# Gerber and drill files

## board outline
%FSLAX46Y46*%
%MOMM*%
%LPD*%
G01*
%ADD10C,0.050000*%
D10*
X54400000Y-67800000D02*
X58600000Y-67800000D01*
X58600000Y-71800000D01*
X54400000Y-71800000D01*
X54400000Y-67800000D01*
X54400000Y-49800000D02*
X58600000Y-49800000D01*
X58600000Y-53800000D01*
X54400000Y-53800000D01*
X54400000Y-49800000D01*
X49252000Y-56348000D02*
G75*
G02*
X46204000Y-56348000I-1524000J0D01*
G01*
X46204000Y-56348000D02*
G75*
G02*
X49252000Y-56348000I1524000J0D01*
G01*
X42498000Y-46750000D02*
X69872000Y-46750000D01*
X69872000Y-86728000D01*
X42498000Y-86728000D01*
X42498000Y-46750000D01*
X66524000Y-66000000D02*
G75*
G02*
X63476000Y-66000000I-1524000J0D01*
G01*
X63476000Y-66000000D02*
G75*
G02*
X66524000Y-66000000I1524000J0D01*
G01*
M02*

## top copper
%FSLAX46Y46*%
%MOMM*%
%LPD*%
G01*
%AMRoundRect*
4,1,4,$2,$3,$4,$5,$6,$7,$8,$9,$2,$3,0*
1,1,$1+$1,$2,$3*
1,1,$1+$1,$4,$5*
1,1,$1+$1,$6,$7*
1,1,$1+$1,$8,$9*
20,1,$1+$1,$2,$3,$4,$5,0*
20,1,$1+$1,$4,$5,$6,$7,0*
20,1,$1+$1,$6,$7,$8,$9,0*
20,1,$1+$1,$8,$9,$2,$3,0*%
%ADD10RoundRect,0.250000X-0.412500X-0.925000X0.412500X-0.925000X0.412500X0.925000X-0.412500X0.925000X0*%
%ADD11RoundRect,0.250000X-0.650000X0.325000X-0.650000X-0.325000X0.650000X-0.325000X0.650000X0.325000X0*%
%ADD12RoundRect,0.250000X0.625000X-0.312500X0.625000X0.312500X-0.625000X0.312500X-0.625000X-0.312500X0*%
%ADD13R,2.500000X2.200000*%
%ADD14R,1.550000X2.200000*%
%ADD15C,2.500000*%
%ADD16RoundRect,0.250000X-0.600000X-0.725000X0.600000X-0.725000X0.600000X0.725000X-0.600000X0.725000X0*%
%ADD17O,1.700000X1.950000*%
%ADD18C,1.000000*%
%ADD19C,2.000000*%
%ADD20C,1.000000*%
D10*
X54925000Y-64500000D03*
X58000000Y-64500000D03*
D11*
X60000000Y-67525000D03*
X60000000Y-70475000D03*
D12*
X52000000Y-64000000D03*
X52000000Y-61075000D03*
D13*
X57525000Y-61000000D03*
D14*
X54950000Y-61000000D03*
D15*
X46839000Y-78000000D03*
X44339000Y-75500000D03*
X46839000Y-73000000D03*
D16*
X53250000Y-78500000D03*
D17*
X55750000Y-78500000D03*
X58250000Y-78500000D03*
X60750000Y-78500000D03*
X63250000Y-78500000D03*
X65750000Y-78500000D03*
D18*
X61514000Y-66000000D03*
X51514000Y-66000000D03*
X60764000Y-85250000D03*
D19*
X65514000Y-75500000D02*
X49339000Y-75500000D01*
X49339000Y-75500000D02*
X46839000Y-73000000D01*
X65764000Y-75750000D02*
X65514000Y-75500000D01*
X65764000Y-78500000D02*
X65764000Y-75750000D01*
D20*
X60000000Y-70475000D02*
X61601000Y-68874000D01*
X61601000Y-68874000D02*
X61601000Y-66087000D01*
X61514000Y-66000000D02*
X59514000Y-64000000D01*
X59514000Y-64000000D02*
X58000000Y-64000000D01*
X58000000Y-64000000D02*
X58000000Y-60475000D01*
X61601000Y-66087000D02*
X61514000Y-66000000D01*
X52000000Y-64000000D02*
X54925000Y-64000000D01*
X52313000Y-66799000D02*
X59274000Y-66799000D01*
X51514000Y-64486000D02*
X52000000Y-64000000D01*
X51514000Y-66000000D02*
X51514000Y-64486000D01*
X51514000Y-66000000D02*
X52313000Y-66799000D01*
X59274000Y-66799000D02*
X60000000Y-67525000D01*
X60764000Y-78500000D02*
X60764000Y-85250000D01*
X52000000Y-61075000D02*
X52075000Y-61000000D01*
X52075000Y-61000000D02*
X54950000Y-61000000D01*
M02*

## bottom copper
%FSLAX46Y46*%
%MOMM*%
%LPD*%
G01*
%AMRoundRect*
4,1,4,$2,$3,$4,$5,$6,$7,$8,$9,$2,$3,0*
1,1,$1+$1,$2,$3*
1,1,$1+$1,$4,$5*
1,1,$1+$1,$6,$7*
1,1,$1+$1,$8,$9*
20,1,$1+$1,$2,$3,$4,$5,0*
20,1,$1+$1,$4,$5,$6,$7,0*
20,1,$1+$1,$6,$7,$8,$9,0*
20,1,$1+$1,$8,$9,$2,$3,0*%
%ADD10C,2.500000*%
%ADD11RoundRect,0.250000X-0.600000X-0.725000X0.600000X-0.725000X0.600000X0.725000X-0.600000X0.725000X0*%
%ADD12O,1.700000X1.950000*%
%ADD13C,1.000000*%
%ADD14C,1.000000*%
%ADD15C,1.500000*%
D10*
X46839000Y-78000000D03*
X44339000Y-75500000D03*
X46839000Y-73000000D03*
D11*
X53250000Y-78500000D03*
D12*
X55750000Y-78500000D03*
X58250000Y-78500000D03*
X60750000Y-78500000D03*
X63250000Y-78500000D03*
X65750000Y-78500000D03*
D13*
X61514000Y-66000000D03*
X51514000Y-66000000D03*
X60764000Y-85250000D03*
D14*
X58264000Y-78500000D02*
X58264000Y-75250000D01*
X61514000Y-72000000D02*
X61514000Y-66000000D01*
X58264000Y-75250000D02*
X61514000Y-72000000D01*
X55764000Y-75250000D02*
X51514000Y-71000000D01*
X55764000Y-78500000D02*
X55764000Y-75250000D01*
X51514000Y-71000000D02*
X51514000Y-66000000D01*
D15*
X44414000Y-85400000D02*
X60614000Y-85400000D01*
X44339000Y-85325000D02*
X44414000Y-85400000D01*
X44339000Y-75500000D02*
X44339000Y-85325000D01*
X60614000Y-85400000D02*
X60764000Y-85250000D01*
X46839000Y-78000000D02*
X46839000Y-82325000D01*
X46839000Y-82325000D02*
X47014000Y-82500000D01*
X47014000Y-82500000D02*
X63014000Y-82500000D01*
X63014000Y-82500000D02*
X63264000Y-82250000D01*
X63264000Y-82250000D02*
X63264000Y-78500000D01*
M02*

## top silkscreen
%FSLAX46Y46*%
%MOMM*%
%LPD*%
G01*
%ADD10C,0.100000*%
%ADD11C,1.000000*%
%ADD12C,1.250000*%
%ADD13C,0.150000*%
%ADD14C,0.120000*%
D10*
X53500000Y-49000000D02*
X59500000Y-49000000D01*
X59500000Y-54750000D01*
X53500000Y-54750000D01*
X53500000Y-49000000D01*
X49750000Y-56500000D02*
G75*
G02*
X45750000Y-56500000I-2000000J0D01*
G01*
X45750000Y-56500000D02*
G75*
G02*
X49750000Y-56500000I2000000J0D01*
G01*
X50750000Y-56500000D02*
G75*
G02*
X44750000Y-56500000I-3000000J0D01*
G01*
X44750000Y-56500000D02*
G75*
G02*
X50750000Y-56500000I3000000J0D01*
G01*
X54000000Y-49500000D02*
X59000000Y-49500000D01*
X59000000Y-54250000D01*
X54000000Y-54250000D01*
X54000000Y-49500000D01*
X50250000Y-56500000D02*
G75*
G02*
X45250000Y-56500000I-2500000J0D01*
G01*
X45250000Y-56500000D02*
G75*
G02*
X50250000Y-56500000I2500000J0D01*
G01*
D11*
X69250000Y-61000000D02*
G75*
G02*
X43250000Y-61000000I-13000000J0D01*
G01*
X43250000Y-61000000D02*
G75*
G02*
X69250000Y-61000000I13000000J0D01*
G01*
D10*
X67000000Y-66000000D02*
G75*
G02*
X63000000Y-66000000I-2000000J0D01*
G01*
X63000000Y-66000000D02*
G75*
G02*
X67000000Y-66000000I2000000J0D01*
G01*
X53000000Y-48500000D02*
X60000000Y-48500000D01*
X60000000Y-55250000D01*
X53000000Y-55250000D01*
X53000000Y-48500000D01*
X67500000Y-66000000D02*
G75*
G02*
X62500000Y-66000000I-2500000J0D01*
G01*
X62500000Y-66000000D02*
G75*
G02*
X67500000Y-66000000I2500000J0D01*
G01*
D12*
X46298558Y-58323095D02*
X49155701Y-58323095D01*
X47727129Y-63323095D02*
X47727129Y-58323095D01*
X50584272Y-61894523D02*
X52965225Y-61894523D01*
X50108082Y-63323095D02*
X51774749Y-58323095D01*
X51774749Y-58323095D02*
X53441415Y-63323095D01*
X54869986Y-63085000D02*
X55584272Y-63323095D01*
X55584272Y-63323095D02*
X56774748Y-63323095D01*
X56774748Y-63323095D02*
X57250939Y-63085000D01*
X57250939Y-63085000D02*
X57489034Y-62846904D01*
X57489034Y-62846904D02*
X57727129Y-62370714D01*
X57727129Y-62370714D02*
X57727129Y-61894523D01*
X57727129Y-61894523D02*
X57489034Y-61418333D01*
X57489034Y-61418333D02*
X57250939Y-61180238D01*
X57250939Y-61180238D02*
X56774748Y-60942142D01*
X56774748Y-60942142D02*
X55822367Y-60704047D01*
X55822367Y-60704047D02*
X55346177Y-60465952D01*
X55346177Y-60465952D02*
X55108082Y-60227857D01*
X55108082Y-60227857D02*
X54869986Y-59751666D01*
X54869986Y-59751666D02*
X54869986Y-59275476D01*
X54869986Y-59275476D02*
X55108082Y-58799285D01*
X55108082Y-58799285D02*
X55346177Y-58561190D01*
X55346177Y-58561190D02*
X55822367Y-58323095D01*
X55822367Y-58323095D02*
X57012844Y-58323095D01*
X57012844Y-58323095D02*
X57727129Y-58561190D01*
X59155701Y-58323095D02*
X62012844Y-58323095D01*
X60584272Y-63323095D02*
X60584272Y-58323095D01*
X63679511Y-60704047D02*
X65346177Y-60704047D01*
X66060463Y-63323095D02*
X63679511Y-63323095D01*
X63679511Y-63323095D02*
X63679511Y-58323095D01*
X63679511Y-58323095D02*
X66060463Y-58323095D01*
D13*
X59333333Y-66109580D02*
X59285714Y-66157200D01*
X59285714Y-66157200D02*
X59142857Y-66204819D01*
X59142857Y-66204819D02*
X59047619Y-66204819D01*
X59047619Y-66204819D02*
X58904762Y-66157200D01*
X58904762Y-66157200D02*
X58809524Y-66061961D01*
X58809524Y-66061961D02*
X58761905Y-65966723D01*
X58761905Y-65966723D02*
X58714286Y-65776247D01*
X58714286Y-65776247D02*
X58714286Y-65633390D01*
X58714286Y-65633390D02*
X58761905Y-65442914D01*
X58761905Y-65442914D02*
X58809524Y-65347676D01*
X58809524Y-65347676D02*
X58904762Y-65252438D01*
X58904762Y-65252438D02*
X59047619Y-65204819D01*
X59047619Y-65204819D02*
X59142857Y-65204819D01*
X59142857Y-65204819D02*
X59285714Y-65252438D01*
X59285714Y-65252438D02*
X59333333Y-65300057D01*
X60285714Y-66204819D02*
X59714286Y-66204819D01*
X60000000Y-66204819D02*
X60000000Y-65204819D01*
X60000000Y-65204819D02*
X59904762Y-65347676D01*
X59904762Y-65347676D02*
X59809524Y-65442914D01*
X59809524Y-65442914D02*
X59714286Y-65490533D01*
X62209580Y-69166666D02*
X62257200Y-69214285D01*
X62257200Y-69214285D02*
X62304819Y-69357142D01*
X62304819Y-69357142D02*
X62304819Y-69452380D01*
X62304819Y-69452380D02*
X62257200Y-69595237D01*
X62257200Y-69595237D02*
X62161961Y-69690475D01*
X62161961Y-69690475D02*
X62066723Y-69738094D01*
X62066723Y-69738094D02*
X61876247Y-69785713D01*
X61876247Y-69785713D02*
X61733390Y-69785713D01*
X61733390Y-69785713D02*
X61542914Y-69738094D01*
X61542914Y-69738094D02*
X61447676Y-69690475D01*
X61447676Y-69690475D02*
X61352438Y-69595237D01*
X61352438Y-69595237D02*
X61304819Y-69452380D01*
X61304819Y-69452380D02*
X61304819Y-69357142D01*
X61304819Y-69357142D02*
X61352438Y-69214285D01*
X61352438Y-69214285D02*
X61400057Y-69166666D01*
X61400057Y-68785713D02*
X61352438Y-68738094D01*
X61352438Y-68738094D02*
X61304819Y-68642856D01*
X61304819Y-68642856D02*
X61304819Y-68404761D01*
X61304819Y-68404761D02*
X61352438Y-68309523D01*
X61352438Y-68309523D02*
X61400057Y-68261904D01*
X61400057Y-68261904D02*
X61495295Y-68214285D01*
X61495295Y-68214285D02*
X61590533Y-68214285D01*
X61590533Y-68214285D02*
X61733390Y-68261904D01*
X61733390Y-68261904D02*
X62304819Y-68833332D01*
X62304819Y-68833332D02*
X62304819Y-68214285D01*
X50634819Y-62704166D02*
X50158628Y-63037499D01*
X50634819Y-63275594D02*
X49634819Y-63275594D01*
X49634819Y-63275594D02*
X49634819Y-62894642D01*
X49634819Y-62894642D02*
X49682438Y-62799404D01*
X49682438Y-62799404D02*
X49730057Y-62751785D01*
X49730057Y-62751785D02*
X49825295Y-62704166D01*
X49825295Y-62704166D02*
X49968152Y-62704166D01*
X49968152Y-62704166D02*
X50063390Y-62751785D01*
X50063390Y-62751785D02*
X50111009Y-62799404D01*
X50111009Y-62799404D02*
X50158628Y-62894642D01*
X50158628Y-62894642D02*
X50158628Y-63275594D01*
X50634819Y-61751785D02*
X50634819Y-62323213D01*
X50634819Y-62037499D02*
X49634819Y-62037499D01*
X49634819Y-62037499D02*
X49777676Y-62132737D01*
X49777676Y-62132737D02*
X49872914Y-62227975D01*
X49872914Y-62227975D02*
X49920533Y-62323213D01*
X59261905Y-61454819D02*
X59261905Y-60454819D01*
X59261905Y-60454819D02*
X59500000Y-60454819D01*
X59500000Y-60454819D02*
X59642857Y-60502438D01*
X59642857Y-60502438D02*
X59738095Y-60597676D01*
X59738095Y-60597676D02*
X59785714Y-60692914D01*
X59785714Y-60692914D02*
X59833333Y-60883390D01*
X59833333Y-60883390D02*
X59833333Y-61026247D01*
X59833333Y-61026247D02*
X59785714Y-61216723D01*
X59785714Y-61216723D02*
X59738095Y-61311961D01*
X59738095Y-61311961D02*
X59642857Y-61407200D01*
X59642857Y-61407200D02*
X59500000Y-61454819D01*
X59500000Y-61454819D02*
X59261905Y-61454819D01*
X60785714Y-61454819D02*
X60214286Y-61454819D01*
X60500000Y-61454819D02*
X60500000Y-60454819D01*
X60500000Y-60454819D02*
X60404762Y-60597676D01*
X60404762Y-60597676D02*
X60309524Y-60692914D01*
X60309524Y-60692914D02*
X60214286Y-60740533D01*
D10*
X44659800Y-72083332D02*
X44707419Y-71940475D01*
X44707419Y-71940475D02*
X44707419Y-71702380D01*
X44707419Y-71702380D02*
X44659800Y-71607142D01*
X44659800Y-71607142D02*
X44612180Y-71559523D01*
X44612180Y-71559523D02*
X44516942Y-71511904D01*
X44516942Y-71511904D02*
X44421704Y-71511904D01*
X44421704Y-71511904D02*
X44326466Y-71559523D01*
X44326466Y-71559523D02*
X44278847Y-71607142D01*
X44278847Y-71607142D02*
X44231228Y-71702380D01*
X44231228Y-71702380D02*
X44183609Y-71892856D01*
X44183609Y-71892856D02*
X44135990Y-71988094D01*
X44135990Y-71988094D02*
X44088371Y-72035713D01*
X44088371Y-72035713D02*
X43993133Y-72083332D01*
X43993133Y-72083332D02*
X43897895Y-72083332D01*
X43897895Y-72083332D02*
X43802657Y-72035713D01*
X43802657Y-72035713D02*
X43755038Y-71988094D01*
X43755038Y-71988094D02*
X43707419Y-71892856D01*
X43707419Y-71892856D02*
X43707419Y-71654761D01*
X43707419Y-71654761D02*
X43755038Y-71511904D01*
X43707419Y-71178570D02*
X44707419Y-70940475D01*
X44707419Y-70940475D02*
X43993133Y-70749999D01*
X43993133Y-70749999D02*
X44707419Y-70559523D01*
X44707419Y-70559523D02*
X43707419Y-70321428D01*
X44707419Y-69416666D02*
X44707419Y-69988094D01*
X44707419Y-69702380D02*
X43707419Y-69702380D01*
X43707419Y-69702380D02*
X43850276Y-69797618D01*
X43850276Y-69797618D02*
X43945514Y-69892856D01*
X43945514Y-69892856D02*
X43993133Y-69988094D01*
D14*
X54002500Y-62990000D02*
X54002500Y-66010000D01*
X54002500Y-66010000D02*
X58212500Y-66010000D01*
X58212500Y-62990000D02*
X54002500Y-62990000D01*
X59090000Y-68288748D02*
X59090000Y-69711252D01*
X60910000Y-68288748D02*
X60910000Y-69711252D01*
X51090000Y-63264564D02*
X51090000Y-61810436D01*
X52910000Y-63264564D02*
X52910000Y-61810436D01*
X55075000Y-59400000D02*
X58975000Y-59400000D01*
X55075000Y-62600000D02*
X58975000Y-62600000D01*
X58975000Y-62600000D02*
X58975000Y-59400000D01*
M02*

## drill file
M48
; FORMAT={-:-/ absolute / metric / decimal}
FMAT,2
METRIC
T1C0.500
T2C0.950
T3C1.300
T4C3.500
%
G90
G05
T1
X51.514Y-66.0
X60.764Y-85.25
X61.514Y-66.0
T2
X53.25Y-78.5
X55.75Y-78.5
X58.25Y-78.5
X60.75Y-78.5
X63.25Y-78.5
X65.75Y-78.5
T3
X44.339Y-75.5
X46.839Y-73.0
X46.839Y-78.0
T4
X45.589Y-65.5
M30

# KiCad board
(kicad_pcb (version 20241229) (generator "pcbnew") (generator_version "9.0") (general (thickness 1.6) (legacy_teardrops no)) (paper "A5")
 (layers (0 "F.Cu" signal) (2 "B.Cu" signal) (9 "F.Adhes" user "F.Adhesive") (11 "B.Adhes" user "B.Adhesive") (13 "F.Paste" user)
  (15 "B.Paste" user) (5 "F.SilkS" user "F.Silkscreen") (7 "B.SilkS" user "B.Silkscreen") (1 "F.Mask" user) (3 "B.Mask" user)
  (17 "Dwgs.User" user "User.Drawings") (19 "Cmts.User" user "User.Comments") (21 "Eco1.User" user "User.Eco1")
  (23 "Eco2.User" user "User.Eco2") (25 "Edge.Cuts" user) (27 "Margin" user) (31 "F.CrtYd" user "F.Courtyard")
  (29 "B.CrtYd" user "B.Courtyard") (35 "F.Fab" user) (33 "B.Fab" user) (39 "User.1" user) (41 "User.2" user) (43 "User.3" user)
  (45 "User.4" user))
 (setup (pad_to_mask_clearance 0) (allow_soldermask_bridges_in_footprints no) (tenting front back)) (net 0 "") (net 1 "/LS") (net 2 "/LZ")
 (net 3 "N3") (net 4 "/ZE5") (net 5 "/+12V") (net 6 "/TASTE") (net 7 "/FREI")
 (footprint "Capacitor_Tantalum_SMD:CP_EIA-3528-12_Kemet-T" (layer "F.Cu") (at 56.4625 64.5)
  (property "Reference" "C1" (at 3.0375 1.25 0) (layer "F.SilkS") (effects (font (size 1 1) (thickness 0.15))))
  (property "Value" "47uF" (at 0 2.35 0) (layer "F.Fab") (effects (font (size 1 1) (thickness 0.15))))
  (fp_line (start -2.46 -1.51) (end -2.46 1.51) (stroke (width 0.12) (type solid)) (layer "F.SilkS"))
  (fp_line (start -2.46 1.51) (end 1.75 1.51) (stroke (width 0.12) (type solid)) (layer "F.SilkS"))
  (fp_line (start 1.75 -1.51) (end -2.46 -1.51) (stroke (width 0.12) (type solid)) (layer "F.SilkS"))
  (pad "1" smd roundrect (at -1.5375 0) (size 1.325 2.35) (layers "F.Cu" "F.Mask" "F.Paste") (roundrect_rratio 0.188679) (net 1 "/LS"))
  (pad "2" smd roundrect (at 1.5375 0) (size 1.325 2.35) (layers "F.Cu" "F.Mask" "F.Paste") (roundrect_rratio 0.188679) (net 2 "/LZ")))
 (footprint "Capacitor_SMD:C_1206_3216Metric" (layer "F.Cu") (at 60 69 -90)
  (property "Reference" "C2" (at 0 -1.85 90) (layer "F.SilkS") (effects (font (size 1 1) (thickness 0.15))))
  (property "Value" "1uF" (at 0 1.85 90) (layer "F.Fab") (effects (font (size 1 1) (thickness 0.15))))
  (fp_line (start -0.711252 0.91) (end 0.711252 0.91) (stroke (width 0.12) (type solid)) (layer "F.SilkS"))
  (fp_line (start -0.711252 -0.91) (end 0.711252 -0.91) (stroke (width 0.12) (type solid)) (layer "F.SilkS"))
  (pad "1" smd roundrect (at -1.475 0 270) (size 1.15 1.8) (layers "F.Cu" "F.Mask" "F.Paste") (roundrect_rratio 0.217391) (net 1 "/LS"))
  (pad "2" smd roundrect (at 1.475 0 270) (size 1.15 1.8) (layers "F.Cu" "F.Mask" "F.Paste") (roundrect_rratio 0.217391) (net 2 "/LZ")))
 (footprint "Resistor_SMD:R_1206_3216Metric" (layer "F.Cu") (at 52 62.5375 90)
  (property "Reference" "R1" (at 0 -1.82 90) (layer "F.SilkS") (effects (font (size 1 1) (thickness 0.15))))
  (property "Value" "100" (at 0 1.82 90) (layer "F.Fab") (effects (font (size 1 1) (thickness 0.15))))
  (fp_line (start -0.727064 -0.91) (end 0.727064 -0.91) (stroke (width 0.12) (type solid)) (layer "F.SilkS"))
  (fp_line (start -0.727064 0.91) (end 0.727064 0.91) (stroke (width 0.12) (type solid)) (layer "F.SilkS"))
  (pad "1" smd roundrect (at -1.4625 0 90) (size 1.125 1.75) (layers "F.Cu" "F.Mask" "F.Paste") (roundrect_rratio 0.222222) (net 1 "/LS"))
  (pad "2" smd roundrect (at 1.4625 0 90) (size 1.125 1.75) (layers "F.Cu" "F.Mask" "F.Paste") (roundrect_rratio 0.222222) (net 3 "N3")))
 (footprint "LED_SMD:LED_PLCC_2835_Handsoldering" (layer "F.Cu") (at 56.475 61 180)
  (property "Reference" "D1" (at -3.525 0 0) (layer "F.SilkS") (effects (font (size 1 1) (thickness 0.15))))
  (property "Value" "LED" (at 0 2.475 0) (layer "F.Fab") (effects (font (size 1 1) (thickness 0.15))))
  (fp_line (start 1.4 1.6) (end -2.5 1.6) (stroke (width 0.12) (type solid)) (layer "F.SilkS"))
  (fp_line (start 1.4 -1.6) (end -2.5 -1.6) (stroke (width 0.12) (type solid)) (layer "F.SilkS"))
  (fp_line (start -2.5 -1.6) (end -2.5 1.6) (stroke (width 0.12) (type solid)) (layer "F.SilkS"))
  (pad "1" smd rect (at -1.05 0 180) (size 2.5 2.2) (layers "F.Cu" "F.Mask" "F.Paste") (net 2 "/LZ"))
  (pad "2" smd rect (at 1.525 0 180) (size 1.55 2.2) (layers "F.Cu" "F.Mask" "F.Paste") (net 3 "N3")))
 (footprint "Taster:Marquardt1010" (layer "F.Cu") (at 45.589 73 90)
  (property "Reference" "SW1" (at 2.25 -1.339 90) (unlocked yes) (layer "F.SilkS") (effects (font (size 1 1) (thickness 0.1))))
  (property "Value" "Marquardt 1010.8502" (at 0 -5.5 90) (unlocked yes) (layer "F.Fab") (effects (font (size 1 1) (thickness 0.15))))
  (pad "" np_thru_hole circle (at 7.5 0 90) (size 3.5 3.5) (drill 3.5) (layers))
  (pad "1" thru_hole circle (at -5 1.25 90) (size 2.5 2.5) (drill 1.3) (layers "*.Cu" "*.Mask") (remove_unused_layers no) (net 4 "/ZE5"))
  (pad "2" thru_hole circle (at -2.5 -1.25 90) (size 2.5 2.5) (drill 1.3) (layers "*.Cu" "*.Mask") (remove_unused_layers no) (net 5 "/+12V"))
  (pad "3" thru_hole circle (at 0 1.25 90) (size 2.5 2.5) (drill 1.3) (layers "*.Cu" "*.Mask") (remove_unused_layers no) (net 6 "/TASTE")))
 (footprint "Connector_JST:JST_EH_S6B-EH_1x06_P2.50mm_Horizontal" (layer "B.Cu") (at 53.25 78.5)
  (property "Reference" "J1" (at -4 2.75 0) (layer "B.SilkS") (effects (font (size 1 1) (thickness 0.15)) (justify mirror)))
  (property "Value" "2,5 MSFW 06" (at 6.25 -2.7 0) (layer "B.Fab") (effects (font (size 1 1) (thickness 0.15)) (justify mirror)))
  (pad "1" thru_hole roundrect (at 0 0) (size 1.7 1.95) (drill 0.95) (layers "*.Cu" "*.Mask") (remove_unused_layers no)
   (roundrect_rratio 0.147059) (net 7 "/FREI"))
  (pad "2" thru_hole oval (at 2.5 0) (size 1.7 1.95) (drill 0.95) (layers "*.Cu" "*.Mask") (remove_unused_layers no) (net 1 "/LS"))
  (pad "3" thru_hole oval (at 5 0) (size 1.7 1.95) (drill 0.95) (layers "*.Cu" "*.Mask") (remove_unused_layers no) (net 2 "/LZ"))
  (pad "4" thru_hole oval (at 7.5 0) (size 1.7 1.95) (drill 0.95) (layers "*.Cu" "*.Mask") (remove_unused_layers no) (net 5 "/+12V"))
  (pad "5" thru_hole oval (at 10 0) (size 1.7 1.95) (drill 0.95) (layers "*.Cu" "*.Mask") (remove_unused_layers no) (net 4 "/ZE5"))
  (pad "6" thru_hole oval (at 12.5 0) (size 1.7 1.95) (drill 0.95) (layers "*.Cu" "*.Mask") (remove_unused_layers no) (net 6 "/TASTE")))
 (gr_rect (start 53.5 49) (end 59.5 54.75) (stroke (width 0.1) (type default)) (fill no) (layer "F.SilkS"))
 (gr_circle (center 47.75 56.5) (end 49.75 56.5) (stroke (width 0.1) (type default)) (fill no) (layer "F.SilkS"))
 (gr_circle (center 47.75 56.5) (end 50.75 56.5) (stroke (width 0.1) (type default)) (fill no) (layer "F.SilkS"))
 (gr_rect (start 54 49.5) (end 59 54.25) (stroke (width 0.1) (type default)) (fill no) (layer "F.SilkS"))
 (gr_circle (center 47.75 56.5) (end 50.25 56.5) (stroke (width 0.1) (type default)) (fill no) (layer "F.SilkS"))
 (gr_circle (center 56.25 61) (end 69.25 61) (stroke (width 1) (type solid)) (fill no) (layer "F.SilkS"))
 (gr_circle (center 65 66) (end 67 66) (stroke (width 0.1) (type default)) (fill no) (layer "F.SilkS"))
 (gr_rect (start 53 48.5) (end 60 55.25) (stroke (width 0.1) (type default)) (fill no) (layer "F.SilkS"))
 (gr_circle (center 65 66) (end 67.5 66) (stroke (width 0.1) (type default)) (fill no) (layer "F.SilkS"))
 (gr_rect (start 54.4 67.8) (end 58.6 71.8) (stroke (width 0.05) (type default)) (fill no) (layer "Edge.Cuts"))
 (gr_rect (start 54.4 49.8) (end 58.6 53.8) (stroke (width 0.05) (type default)) (fill no) (layer "Edge.Cuts"))
 (gr_circle (center 47.728 56.348) (end 49.252 56.348) (stroke (width 0.05) (type default)) (fill no) (layer "Edge.Cuts"))
 (gr_rect (start 42.498 46.75) (end 69.872 86.728) (stroke (width 0.05) (type default)) (fill no) (layer "Edge.Cuts"))
 (gr_circle (center 65 66) (end 66.524 66) (stroke (width 0.05) (type default)) (fill no) (layer "Edge.Cuts"))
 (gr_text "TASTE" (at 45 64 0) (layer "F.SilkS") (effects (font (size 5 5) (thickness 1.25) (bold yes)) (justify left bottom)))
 (segment (start 65.514 75.5) (end 49.339 75.5) (width 2) (layer "F.Cu") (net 6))
 (segment (start 49.339 75.5) (end 46.839 73) (width 2) (layer "F.Cu") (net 6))
 (segment (start 65.764 75.75) (end 65.514 75.5) (width 2) (layer "F.Cu") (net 6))
 (segment (start 65.764 78.5) (end 65.764 75.75) (width 2) (layer "F.Cu") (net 6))
 (segment (start 60 70.475) (end 61.601 68.874) (width 1) (layer "F.Cu") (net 2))
 (segment (start 61.601 68.874) (end 61.601 66.087) (width 1) (layer "F.Cu") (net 2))
 (segment (start 61.514 66) (end 59.514 64) (width 1) (layer "F.Cu") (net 2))
 (segment (start 59.514 64) (end 58 64) (width 1) (layer "F.Cu") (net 2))
 (segment (start 58 64) (end 58 60.475) (width 1) (layer "F.Cu") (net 2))
 (segment (start 61.601 66.087) (end 61.514 66) (width 1) (layer "F.Cu") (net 2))
 (via (at 61.514 66) (size 1) (drill 0.5) (layers "F.Cu" "B.Cu") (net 2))
 (segment (start 58.264 78.5) (end 58.264 75.25) (width 1) (layer "B.Cu") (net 2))
 (segment (start 61.514 72) (end 61.514 66) (width 1) (layer "B.Cu") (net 2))
 (segment (start 58.264 75.25) (end 61.514 72) (width 1) (layer "B.Cu") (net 2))
 (segment (start 52 64) (end 54.925 64) (width 1) (layer "F.Cu") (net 1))
 (segment (start 52.313 66.799) (end 59.274 66.799) (width 1) (layer "F.Cu") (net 1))
 (segment (start 51.514 64.486) (end 52 64) (width 1) (layer "F.Cu") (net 1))
 (segment (start 51.514 66) (end 51.514 64.486) (width 1) (layer "F.Cu") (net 1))
 (segment (start 51.514 66) (end 52.313 66.799) (width 1) (layer "F.Cu") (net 1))
 (segment (start 59.274 66.799) (end 60 67.525) (width 1) (layer "F.Cu") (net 1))
 (via (at 51.514 66) (size 1) (drill 0.5) (layers "F.Cu" "B.Cu") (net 1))
 (segment (start 55.764 75.25) (end 51.514 71) (width 1) (layer "B.Cu") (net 1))
 (segment (start 55.764 78.5) (end 55.764 75.25) (width 1) (layer "B.Cu") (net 1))
 (segment (start 51.514 71) (end 51.514 66) (width 1) (layer "B.Cu") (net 1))
 (segment (start 60.764 78.5) (end 60.764 85.25) (width 1) (layer "F.Cu") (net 5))
 (via (at 60.764 85.25) (size 1) (drill 0.5) (layers "F.Cu" "B.Cu") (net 5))
 (segment (start 44.414 85.4) (end 60.614 85.4) (width 1.5) (layer "B.Cu") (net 5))
 (segment (start 44.339 85.325) (end 44.414 85.4) (width 1.5) (layer "B.Cu") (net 5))
 (segment (start 44.339 75.5) (end 44.339 85.325) (width 1.5) (layer "B.Cu") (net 5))
 (segment (start 60.614 85.4) (end 60.764 85.25) (width 1.5) (layer "B.Cu") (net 5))
 (segment (start 46.839 78) (end 46.839 82.325) (width 1.5) (layer "B.Cu") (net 4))
 (segment (start 46.839 82.325) (end 47.014 82.5) (width 1.5) (layer "B.Cu") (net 4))
 (segment (start 47.014 82.5) (end 63.014 82.5) (width 1.5) (layer "B.Cu") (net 4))
 (segment (start 63.014 82.5) (end 63.264 82.25) (width 1.5) (layer "B.Cu") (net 4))
 (segment (start 63.264 82.25) (end 63.264 78.5) (width 1.5) (layer "B.Cu") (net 4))
 (segment (start 52 61.075) (end 52.075 61) (width 1) (layer "F.Cu") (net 3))
 (segment (start 52.075 61) (end 54.95 61) (width 1) (layer "F.Cu") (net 3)))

